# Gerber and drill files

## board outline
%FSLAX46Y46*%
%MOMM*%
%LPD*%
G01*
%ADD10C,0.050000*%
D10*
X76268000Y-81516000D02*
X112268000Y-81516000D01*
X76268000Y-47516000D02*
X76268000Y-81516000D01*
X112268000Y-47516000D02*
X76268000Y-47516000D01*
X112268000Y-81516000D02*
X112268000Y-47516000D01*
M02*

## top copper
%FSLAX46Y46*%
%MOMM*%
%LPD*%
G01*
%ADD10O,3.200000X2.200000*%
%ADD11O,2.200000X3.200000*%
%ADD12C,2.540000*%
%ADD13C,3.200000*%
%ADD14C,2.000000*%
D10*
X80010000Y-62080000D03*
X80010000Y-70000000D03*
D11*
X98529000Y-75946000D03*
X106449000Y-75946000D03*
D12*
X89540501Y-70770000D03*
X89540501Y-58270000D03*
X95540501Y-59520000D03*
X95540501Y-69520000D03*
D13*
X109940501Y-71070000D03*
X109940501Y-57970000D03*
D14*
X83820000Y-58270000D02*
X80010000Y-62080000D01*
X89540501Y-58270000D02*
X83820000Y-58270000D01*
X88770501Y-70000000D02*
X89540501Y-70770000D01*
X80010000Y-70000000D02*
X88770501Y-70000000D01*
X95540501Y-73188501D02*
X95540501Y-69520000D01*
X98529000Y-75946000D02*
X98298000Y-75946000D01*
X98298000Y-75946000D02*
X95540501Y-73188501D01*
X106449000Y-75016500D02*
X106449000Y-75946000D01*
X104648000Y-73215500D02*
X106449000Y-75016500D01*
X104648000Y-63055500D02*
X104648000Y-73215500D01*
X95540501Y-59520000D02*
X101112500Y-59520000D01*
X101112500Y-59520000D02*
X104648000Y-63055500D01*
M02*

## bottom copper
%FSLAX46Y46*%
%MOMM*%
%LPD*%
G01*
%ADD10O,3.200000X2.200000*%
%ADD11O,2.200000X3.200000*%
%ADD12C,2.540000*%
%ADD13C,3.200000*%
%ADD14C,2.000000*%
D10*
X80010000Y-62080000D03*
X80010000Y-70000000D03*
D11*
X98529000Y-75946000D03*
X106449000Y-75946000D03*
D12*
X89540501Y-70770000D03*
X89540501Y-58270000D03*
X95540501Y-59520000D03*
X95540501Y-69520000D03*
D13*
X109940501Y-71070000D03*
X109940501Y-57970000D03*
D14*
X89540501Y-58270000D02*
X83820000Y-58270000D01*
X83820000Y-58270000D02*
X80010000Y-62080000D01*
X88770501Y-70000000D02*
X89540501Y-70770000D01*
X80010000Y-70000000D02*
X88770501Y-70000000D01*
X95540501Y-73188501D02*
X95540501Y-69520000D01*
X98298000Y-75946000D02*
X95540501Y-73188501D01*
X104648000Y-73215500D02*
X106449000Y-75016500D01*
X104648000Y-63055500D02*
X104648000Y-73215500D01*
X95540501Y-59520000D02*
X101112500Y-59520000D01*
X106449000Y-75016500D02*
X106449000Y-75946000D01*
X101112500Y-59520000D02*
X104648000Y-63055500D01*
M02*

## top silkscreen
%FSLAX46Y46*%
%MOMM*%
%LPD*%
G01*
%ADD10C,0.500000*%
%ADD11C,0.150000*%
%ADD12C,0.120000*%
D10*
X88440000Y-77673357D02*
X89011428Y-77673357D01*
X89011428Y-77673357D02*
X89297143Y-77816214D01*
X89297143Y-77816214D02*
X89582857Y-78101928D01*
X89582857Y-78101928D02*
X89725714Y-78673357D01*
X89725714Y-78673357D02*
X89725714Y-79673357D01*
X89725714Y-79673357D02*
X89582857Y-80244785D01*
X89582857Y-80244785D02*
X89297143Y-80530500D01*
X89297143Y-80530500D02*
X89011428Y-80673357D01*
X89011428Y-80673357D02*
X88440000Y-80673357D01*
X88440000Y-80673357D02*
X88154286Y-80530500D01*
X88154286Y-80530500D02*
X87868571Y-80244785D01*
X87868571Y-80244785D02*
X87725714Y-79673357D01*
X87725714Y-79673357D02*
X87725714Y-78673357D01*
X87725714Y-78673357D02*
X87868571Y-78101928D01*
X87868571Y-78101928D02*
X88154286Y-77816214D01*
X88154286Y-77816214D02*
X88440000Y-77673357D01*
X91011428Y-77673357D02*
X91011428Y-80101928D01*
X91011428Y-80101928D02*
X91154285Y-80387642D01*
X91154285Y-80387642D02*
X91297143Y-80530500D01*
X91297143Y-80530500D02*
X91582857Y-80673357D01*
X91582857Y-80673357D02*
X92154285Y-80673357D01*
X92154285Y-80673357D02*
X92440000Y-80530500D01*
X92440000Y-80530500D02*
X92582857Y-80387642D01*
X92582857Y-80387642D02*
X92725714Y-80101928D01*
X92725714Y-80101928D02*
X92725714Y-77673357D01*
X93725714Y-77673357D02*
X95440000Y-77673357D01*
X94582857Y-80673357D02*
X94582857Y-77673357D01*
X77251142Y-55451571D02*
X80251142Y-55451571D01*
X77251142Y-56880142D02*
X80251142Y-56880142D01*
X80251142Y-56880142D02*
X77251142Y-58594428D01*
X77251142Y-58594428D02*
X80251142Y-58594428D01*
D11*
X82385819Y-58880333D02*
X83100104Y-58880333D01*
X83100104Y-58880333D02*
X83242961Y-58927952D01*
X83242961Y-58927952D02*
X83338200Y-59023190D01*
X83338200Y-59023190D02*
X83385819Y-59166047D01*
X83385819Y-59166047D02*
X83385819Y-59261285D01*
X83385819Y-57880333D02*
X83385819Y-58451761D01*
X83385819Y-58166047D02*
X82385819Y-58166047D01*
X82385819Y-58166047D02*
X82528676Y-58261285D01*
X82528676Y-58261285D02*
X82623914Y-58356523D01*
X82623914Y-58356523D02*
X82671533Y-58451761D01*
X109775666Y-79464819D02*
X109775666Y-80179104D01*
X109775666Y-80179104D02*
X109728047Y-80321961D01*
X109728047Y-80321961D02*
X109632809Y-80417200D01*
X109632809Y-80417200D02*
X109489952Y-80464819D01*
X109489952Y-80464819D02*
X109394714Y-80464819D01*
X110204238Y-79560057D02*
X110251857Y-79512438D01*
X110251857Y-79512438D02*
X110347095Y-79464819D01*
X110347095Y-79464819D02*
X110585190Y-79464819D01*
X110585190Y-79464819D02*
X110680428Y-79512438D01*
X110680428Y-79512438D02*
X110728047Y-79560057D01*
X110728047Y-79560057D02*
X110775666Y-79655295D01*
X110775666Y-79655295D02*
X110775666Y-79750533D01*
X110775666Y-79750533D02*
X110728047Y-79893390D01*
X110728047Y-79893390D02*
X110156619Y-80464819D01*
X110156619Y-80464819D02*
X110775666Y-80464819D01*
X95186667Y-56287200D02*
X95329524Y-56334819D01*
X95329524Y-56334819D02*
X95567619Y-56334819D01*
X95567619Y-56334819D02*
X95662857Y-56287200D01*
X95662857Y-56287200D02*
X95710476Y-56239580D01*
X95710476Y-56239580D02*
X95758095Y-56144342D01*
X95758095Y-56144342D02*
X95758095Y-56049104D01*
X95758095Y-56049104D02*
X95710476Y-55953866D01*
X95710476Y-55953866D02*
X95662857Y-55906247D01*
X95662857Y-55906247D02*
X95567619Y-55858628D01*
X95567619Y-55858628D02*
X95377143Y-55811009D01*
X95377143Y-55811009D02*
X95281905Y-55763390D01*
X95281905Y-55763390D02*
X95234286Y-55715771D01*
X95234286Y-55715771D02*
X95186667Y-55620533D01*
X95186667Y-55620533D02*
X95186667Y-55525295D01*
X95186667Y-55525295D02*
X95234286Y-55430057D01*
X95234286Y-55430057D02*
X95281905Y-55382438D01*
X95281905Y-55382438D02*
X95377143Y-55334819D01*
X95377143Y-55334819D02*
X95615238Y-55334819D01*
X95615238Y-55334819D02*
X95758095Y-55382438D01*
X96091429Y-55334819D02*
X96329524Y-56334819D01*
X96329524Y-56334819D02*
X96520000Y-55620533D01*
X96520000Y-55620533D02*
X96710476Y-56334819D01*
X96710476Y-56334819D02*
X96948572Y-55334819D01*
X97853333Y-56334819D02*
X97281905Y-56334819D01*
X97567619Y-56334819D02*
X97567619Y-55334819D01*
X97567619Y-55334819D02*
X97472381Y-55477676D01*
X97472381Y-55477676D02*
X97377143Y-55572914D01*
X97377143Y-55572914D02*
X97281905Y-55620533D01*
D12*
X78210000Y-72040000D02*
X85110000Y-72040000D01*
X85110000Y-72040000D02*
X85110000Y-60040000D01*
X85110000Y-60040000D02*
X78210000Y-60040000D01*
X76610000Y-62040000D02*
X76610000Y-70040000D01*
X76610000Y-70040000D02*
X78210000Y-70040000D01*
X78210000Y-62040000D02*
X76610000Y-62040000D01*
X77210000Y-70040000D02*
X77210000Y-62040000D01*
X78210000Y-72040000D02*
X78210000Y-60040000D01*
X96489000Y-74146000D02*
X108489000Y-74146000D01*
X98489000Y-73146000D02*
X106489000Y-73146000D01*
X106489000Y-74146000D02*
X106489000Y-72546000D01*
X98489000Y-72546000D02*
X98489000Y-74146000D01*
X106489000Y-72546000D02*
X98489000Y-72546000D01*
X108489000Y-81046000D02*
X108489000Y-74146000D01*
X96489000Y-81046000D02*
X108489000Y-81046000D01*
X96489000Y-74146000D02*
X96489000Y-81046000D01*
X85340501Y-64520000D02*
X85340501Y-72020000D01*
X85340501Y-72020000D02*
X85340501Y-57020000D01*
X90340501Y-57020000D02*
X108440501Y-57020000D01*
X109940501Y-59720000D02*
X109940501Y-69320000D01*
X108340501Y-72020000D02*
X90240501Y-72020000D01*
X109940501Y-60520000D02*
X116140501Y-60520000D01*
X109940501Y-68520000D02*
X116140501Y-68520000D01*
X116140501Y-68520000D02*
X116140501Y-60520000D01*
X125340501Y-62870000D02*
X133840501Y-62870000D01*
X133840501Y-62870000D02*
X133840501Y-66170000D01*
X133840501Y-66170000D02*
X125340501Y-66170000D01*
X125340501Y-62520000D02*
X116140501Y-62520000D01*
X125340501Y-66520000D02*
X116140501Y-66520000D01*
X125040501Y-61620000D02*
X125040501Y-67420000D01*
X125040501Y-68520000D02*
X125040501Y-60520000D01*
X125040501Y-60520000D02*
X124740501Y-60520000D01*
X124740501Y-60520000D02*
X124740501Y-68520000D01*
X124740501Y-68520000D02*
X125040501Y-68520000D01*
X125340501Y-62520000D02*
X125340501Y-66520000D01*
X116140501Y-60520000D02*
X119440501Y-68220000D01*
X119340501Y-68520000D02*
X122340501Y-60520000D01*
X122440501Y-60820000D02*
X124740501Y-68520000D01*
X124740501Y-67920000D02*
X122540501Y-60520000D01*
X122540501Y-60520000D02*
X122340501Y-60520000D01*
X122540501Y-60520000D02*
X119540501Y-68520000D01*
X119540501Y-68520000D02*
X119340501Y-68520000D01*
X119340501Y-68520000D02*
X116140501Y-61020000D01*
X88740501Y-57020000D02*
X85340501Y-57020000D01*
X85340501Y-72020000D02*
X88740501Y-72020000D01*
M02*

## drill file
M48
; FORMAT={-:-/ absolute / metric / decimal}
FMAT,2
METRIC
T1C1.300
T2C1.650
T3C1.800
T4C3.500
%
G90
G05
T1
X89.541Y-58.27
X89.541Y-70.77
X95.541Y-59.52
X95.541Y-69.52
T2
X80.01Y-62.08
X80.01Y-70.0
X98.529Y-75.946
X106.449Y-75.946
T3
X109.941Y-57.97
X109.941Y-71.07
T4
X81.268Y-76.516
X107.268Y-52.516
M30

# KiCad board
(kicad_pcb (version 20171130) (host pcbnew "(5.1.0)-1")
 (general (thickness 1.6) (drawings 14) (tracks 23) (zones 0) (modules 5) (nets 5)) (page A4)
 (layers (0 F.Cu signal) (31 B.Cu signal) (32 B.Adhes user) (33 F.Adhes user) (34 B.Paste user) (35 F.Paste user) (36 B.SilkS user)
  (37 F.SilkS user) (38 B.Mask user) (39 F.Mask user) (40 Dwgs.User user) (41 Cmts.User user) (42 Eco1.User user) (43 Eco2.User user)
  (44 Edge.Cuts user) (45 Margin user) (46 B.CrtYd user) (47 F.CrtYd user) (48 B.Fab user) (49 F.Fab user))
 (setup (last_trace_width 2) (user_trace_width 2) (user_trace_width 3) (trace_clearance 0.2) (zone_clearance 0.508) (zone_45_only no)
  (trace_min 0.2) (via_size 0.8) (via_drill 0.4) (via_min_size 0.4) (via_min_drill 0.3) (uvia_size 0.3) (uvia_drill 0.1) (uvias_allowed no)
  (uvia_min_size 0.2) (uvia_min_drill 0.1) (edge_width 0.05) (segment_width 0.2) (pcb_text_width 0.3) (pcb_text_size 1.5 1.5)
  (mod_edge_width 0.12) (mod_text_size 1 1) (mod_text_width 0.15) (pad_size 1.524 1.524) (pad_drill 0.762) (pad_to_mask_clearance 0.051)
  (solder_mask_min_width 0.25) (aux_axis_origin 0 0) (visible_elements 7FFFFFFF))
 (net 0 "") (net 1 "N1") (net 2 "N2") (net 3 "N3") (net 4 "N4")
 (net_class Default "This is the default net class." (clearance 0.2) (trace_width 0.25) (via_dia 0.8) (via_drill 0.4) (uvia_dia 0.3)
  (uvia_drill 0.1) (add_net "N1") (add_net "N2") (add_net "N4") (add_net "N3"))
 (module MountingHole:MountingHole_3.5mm (layer F.Cu) (at 107.268 52.516)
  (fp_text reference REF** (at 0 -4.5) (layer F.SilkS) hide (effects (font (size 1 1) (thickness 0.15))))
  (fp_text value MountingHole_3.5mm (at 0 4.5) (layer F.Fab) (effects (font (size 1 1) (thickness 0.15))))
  (pad 1 np_thru_hole circle (at 0 0) (size 3.5 3.5) (drill 3.5) (layers *.Cu *.Mask)))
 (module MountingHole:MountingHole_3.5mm (layer F.Cu) (at 81.268 76.516)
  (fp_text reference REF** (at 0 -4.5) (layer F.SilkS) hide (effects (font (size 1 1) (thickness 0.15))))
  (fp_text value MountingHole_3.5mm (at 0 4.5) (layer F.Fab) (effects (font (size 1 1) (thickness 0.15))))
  (pad 1 np_thru_hole circle (at 0 0) (size 3.5 3.5) (drill 3.5) (layers *.Cu *.Mask)))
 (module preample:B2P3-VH (layer F.Cu) (at 80.01 66.04 270)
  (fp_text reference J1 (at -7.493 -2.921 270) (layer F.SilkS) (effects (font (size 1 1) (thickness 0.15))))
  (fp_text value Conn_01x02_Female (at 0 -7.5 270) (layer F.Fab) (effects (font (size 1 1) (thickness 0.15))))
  (fp_line (start 6 1.8) (end 6 -5.1) (layer F.SilkS) (width 0.12))
  (fp_line (start 6 -5.1) (end -6 -5.1) (layer F.SilkS) (width 0.12))
  (fp_line (start -6 -5.1) (end -6 1.8) (layer F.SilkS) (width 0.12))
  (fp_line (start -4 3.4) (end 4 3.4) (layer F.SilkS) (width 0.12))
  (fp_line (start 4 3.4) (end 4 1.8) (layer F.SilkS) (width 0.12))
  (fp_line (start -4 1.8) (end -4 3.4) (layer F.SilkS) (width 0.12))
  (fp_line (start 4 2.8) (end -4 2.8) (layer F.SilkS) (width 0.12))
  (fp_line (start 6 1.8) (end -6 1.8) (layer F.SilkS) (width 0.12))
  (pad 1 thru_hole oval (at -3.96 0 270) (size 2.2 3.2) (drill 1.65) (layers *.Cu *.Mask) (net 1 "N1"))
  (pad 2 thru_hole oval (at 3.96 0 270) (size 2.2 3.2) (drill 1.65) (layers *.Cu *.Mask) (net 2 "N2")))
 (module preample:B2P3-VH (layer F.Cu) (at 102.489 75.946 180)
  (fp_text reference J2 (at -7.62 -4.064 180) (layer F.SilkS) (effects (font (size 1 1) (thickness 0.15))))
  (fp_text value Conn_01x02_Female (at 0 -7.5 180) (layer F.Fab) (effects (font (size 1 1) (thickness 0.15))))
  (fp_line (start 6 1.8) (end -6 1.8) (layer F.SilkS) (width 0.12))
  (fp_line (start 4 2.8) (end -4 2.8) (layer F.SilkS) (width 0.12))
  (fp_line (start -4 1.8) (end -4 3.4) (layer F.SilkS) (width 0.12))
  (fp_line (start 4 3.4) (end 4 1.8) (layer F.SilkS) (width 0.12))
  (fp_line (start -4 3.4) (end 4 3.4) (layer F.SilkS) (width 0.12))
  (fp_line (start -6 -5.1) (end -6 1.8) (layer F.SilkS) (width 0.12))
  (fp_line (start 6 -5.1) (end -6 -5.1) (layer F.SilkS) (width 0.12))
  (fp_line (start 6 1.8) (end 6 -5.1) (layer F.SilkS) (width 0.12))
  (pad 2 thru_hole oval (at 3.96 0 180) (size 2.2 3.2) (drill 1.65) (layers *.Cu *.Mask) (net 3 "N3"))
  (pad 1 thru_hole oval (at -3.96 0 180) (size 2.2 3.2) (drill 1.65) (layers *.Cu *.Mask) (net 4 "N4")))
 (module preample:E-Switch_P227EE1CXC (layer F.Cu) (at 99.740501 64.52)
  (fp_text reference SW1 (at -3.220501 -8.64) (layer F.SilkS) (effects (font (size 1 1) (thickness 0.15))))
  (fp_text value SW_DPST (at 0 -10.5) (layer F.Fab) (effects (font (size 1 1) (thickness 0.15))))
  (fp_line (start -14.4 0) (end -14.4 7.5) (layer F.SilkS) (width 0.12))
  (fp_line (start -14.4 7.5) (end -14.4 -7.5) (layer F.SilkS) (width 0.12))
  (fp_line (start -9.4 -7.5) (end 8.7 -7.5) (layer F.SilkS) (width 0.12))
  (fp_line (start 10.2 -4.8) (end 10.2 4.8) (layer F.SilkS) (width 0.12))
  (fp_line (start 8.6 7.5) (end -9.5 7.5) (layer F.SilkS) (width 0.12))
  (fp_line (start 10.2 -4) (end 16.4 -4) (layer F.SilkS) (width 0.12))
  (fp_line (start 10.2 4) (end 16.4 4) (layer F.SilkS) (width 0.12))
  (fp_line (start 16.4 4) (end 16.4 -4) (layer F.SilkS) (width 0.12))
  (fp_line (start 25.6 -1.65) (end 34.1 -1.65) (layer F.SilkS) (width 0.12))
  (fp_line (start 34.1 -1.65) (end 34.1 1.65) (layer F.SilkS) (width 0.12))
  (fp_line (start 34.1 1.65) (end 25.6 1.65) (layer F.SilkS) (width 0.12))
  (fp_line (start 25.6 -2) (end 16.4 -2) (layer F.SilkS) (width 0.12))
  (fp_line (start 25.6 2) (end 16.4 2) (layer F.SilkS) (width 0.12))
  (fp_line (start 25.3 -2.9) (end 25.3 2.9) (layer F.SilkS) (width 0.12))
  (fp_line (start 25.3 4) (end 25.3 -4) (layer F.SilkS) (width 0.12))
  (fp_line (start 25.3 -4) (end 25 -4) (layer F.SilkS) (width 0.12))
  (fp_line (start 25 -4) (end 25 4) (layer F.SilkS) (width 0.12))
  (fp_line (start 25 4) (end 25.3 4) (layer F.SilkS) (width 0.12))
  (fp_line (start 25.6 -2) (end 25.6 2) (layer F.SilkS) (width 0.12))
  (fp_line (start 16.4 -4) (end 19.7 3.7) (layer F.SilkS) (width 0.12))
  (fp_line (start 19.6 4) (end 22.6 -4) (layer F.SilkS) (width 0.12))
  (fp_line (start 22.7 -3.7) (end 25 4) (layer F.SilkS) (width 0.12))
  (fp_line (start 25 3.4) (end 22.8 -4) (layer F.SilkS) (width 0.12))
  (fp_line (start 22.8 -4) (end 22.6 -4) (layer F.SilkS) (width 0.12))
  (fp_line (start 22.8 -4) (end 19.8 4) (layer F.SilkS) (width 0.12))
  (fp_line (start 19.8 4) (end 19.6 4) (layer F.SilkS) (width 0.12))
  (fp_line (start 19.6 4) (end 16.4 -3.5) (layer F.SilkS) (width 0.12))
  (fp_line (start -11 -7.5) (end -14.4 -7.5) (layer F.SilkS) (width 0.12))
  (fp_line (start -14.4 7.5) (end -11 7.5) (layer F.SilkS) (width 0.12))
  (pad 3 thru_hole circle (at -10.2 6.25) (size 2.54 2.54) (drill 1.3) (layers *.Cu *.Mask) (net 2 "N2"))
  (pad 1 thru_hole circle (at -10.2 -6.25) (size 2.54 2.54) (drill 1.3) (layers *.Cu *.Mask) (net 1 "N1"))
  (pad 2 thru_hole circle (at -4.2 -5) (size 2.54 2.54) (drill 1.3) (layers *.Cu *.Mask) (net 4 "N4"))
  (pad 4 thru_hole circle (at -4.2 5) (size 2.54 2.54) (drill 1.3) (layers *.Cu *.Mask) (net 3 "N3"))
  (pad 0 thru_hole circle (at 10.2 6.55) (size 3.2 3.2) (drill 1.8) (layers *.Cu *.Mask))
  (pad 0 thru_hole circle (at 10.2 -6.55) (size 3.2 3.2) (drill 1.8) (layers *.Cu *.Mask)))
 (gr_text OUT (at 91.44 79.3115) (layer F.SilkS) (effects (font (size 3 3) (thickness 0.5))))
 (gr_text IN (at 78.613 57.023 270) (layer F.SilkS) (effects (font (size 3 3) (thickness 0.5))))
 (gr_line (start 76.268 81.516) (end 112.268 81.516) (layer Edge.Cuts) (width 0.05))
 (gr_line (start 76.268 47.516) (end 76.268 81.516) (layer Edge.Cuts) (width 0.05))
 (gr_line (start 112.268 47.516) (end 76.268 47.516) (layer Edge.Cuts) (width 0.05))
 (gr_line (start 112.268 81.516) (end 112.268 47.516) (layer Edge.Cuts) (width 0.05))
 (segment (start 89.540501 58.27) (end 83.82 58.27) (width 2) (layer B.Cu) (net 1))
 (segment (start 83.82 58.27) (end 80.01 62.08) (width 2) (layer B.Cu) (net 1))
 (segment (start 88.770501 70) (end 89.540501 70.77) (width 2) (layer B.Cu) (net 2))
 (segment (start 80.01 70) (end 88.770501 70) (width 2) (layer B.Cu) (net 2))
 (segment (start 95.540501 73.188501) (end 95.540501 69.52) (width 2) (layer B.Cu) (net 3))
 (segment (start 98.298 75.946) (end 95.540501 73.188501) (width 2) (layer B.Cu) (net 3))
 (segment (start 104.648 73.2155) (end 106.449 75.0165) (width 2) (layer B.Cu) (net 4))
 (segment (start 104.648 63.0555) (end 104.648 73.2155) (width 2) (layer B.Cu) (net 4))
 (segment (start 95.540501 59.52) (end 101.1125 59.52) (width 2) (layer B.Cu) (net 4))
 (segment (start 106.449 75.0165) (end 106.449 75.946) (width 2) (layer B.Cu) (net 4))
 (segment (start 101.1125 59.52) (end 104.648 63.0555) (width 2) (layer B.Cu) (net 4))
 (segment (start 83.82 58.27) (end 80.01 62.08) (width 2) (layer F.Cu) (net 1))
 (segment (start 89.540501 58.27) (end 83.82 58.27) (width 2) (layer F.Cu) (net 1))
 (segment (start 88.770501 70) (end 89.540501 70.77) (width 2) (layer F.Cu) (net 2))
 (segment (start 80.01 70) (end 88.770501 70) (width 2) (layer F.Cu) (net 2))
 (segment (start 95.540501 73.188501) (end 95.540501 69.52) (width 2) (layer F.Cu) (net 3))
 (segment (start 98.529 75.946) (end 98.298 75.946) (width 2) (layer F.Cu) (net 3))
 (segment (start 98.298 75.946) (end 95.540501 73.188501) (width 2) (layer F.Cu) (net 3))
 (segment (start 106.449 75.0165) (end 106.449 75.946) (width 2) (layer F.Cu) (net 4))
 (segment (start 104.648 73.2155) (end 106.449 75.0165) (width 2) (layer F.Cu) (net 4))
 (segment (start 104.648 63.0555) (end 104.648 73.2155) (width 2) (layer F.Cu) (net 4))
 (segment (start 95.540501 59.52) (end 101.1125 59.52) (width 2) (layer F.Cu) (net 4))
 (segment (start 101.1125 59.52) (end 104.648 63.0555) (width 2) (layer F.Cu) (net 4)))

